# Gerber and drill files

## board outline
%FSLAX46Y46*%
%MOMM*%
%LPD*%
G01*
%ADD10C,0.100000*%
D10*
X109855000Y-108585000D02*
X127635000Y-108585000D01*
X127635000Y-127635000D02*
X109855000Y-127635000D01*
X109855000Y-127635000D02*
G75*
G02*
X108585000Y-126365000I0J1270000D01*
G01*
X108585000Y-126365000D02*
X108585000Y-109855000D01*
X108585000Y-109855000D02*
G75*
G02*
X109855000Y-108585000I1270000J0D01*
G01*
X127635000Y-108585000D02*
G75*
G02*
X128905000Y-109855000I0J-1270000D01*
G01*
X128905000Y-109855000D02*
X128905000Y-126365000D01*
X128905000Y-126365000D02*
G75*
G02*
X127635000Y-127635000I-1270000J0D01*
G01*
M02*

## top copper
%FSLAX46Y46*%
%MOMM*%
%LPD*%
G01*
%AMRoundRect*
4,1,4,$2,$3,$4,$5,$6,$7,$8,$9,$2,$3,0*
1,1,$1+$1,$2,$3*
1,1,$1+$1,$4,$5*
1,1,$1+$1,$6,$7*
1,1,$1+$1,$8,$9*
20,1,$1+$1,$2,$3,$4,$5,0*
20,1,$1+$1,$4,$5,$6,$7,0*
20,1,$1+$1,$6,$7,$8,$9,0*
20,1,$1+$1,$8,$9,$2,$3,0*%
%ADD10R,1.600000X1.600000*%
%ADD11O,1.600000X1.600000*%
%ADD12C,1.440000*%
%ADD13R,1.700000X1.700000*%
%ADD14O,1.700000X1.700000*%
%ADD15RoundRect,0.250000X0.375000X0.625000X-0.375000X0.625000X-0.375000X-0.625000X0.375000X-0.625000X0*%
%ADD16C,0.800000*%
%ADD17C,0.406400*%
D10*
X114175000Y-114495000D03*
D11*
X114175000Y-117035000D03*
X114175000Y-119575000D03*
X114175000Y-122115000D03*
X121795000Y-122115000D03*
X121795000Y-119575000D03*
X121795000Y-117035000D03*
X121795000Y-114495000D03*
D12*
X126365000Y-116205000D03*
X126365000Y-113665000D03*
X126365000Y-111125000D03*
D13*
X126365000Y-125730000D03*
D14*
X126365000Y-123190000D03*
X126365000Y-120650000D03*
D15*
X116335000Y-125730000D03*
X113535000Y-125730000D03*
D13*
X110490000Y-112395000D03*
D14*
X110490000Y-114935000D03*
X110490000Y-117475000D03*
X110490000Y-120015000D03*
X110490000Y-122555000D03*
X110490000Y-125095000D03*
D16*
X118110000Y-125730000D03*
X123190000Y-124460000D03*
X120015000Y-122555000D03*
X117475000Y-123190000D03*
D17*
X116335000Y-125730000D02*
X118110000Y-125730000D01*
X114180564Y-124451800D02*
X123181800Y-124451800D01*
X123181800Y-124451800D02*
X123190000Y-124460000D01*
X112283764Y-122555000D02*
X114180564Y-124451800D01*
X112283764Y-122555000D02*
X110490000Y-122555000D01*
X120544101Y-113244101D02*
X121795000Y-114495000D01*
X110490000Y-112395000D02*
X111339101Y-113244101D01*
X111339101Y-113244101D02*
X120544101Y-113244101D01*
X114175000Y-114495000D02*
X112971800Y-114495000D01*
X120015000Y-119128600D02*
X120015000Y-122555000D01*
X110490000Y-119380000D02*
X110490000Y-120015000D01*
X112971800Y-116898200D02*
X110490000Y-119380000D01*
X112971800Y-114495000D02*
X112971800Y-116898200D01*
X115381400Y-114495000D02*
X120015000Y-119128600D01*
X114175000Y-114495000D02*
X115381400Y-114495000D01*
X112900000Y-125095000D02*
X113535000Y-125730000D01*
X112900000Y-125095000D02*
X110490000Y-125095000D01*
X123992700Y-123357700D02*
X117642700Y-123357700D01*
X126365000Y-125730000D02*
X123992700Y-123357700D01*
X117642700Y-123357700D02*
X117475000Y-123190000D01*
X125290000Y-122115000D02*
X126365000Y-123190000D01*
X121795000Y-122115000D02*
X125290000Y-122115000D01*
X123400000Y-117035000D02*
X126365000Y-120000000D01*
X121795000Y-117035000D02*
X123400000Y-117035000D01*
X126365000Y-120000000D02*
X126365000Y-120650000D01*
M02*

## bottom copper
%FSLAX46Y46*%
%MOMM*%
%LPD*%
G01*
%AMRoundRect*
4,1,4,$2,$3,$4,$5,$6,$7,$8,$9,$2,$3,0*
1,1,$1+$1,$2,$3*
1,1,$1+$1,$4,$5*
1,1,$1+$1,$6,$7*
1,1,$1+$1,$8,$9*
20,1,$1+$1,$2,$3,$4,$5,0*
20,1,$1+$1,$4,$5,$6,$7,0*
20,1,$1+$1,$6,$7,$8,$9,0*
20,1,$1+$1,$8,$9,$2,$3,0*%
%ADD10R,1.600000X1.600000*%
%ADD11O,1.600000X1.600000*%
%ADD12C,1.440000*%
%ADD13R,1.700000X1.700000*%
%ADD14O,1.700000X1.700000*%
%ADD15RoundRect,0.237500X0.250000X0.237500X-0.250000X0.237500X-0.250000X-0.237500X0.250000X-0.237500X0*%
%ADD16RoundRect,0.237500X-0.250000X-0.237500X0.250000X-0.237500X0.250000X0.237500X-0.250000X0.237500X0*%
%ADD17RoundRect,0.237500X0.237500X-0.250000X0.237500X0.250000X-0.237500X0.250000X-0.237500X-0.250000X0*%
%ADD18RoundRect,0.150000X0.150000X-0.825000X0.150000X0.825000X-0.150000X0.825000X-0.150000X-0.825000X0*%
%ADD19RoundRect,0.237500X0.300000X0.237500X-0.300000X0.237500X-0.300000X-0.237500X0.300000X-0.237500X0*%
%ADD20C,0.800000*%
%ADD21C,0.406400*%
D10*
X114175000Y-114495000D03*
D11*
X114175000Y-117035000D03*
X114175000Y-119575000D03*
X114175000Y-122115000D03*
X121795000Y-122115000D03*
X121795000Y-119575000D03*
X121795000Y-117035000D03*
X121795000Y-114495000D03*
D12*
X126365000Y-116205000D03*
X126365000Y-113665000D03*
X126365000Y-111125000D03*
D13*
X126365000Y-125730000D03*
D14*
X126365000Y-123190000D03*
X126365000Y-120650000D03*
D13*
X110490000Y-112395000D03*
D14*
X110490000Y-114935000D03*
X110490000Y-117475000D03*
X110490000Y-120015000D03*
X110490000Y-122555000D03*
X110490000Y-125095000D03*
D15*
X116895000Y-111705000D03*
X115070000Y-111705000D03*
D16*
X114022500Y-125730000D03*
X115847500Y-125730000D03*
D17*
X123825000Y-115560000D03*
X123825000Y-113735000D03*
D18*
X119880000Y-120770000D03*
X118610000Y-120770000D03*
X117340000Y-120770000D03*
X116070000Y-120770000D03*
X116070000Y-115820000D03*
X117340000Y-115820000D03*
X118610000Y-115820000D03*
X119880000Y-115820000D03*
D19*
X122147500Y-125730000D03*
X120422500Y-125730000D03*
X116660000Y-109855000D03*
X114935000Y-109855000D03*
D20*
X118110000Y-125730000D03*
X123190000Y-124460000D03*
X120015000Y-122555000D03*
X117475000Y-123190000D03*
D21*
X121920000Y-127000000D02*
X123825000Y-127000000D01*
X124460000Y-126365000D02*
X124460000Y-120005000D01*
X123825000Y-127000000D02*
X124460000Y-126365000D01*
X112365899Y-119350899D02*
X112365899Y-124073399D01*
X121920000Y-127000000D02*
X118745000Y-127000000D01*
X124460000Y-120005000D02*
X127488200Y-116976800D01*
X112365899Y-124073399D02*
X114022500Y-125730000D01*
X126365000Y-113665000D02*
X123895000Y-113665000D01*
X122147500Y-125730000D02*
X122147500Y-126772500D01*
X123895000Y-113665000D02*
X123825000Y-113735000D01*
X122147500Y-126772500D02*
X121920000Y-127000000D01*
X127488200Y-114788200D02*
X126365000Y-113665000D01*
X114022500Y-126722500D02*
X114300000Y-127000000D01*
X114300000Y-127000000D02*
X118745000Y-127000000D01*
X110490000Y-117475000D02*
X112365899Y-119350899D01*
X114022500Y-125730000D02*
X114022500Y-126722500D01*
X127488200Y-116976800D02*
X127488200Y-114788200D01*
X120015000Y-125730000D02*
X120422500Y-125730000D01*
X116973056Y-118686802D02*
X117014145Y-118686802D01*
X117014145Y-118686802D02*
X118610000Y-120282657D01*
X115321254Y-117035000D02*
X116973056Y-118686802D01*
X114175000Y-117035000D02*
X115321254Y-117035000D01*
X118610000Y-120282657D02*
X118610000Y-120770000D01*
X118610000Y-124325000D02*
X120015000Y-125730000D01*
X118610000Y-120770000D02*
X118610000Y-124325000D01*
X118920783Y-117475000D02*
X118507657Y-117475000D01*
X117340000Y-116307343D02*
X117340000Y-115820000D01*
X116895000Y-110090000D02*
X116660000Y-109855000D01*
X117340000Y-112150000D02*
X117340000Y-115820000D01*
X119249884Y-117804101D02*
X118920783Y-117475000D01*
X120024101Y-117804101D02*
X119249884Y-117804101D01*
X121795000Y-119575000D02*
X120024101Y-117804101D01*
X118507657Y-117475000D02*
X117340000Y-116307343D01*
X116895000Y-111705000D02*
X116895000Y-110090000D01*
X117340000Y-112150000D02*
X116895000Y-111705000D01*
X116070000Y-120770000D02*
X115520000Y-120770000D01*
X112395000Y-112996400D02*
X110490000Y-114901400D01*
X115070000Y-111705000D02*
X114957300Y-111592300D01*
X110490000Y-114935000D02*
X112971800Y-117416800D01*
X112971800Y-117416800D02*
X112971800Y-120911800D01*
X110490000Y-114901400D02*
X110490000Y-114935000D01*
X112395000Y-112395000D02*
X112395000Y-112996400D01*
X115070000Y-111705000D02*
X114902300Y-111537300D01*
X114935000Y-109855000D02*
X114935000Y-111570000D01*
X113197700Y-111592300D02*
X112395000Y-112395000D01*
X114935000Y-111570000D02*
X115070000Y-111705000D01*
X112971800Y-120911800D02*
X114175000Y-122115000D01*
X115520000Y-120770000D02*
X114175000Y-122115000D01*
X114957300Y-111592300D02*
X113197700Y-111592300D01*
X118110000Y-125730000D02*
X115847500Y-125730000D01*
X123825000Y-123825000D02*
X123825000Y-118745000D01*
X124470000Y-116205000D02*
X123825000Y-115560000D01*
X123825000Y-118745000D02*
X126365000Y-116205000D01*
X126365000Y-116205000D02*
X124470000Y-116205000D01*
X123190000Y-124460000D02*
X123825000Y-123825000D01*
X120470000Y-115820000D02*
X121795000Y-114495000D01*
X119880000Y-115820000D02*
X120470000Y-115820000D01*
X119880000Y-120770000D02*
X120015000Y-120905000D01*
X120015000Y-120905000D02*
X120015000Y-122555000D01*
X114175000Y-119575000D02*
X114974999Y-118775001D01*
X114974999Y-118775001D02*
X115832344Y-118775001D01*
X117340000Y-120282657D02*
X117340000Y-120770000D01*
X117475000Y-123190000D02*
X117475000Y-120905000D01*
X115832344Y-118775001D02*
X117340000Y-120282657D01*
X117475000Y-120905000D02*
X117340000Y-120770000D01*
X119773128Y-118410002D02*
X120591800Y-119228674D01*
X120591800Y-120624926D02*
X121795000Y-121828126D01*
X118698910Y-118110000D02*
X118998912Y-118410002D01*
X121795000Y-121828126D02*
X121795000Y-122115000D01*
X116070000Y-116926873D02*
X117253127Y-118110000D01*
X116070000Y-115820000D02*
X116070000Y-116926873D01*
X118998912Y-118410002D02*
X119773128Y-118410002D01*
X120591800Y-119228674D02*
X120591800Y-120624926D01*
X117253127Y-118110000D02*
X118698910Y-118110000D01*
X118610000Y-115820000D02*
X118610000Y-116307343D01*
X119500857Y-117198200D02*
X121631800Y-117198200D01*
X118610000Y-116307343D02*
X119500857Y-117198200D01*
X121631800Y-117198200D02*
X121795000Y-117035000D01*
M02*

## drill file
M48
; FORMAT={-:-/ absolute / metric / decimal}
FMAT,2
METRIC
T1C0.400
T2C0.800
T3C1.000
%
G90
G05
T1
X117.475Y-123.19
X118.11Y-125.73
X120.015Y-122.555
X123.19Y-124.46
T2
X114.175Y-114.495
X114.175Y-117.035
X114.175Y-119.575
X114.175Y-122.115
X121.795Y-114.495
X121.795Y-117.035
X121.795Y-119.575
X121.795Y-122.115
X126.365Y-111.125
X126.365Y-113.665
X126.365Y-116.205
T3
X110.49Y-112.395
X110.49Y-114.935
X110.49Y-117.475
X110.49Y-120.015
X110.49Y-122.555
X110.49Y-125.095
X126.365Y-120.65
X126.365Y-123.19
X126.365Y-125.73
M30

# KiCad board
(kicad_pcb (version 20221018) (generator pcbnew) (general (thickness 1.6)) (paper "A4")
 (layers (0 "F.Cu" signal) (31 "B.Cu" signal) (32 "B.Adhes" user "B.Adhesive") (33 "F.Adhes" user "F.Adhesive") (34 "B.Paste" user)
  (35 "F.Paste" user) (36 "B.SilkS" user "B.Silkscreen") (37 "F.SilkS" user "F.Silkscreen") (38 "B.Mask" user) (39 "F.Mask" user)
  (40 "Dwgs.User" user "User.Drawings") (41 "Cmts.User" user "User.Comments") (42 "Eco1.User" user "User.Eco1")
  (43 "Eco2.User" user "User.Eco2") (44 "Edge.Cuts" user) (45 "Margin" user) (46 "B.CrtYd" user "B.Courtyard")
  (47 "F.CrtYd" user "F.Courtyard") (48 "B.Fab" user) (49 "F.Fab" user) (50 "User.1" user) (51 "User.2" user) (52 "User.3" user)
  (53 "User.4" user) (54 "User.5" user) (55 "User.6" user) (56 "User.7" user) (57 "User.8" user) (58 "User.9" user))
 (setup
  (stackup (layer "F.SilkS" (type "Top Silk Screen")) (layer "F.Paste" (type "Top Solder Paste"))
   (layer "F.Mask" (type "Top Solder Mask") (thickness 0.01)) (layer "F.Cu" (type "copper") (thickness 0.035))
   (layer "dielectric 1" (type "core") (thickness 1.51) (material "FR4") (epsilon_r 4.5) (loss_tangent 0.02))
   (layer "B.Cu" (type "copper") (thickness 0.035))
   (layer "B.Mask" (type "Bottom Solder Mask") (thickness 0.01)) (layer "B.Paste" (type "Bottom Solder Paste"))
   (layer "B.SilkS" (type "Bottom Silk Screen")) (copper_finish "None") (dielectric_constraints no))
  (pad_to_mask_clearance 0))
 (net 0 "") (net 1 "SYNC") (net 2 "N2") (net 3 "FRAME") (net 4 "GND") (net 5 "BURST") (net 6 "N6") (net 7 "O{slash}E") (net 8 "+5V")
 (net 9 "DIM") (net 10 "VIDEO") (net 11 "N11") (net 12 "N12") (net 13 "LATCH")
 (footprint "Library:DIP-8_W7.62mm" (layer "F.Cu") (at 114.175 114.495)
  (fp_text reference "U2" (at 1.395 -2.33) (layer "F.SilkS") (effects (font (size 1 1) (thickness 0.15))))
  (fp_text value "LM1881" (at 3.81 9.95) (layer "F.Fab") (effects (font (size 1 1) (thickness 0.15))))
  (pad "1" thru_hole rect (at 0 0) (size 1.6 1.6) (drill 0.8) (layers "*.Cu" "*.Mask") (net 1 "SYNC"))
  (pad "2" thru_hole oval (at 0 2.54) (size 1.6 1.6) (drill 0.8) (layers "*.Cu" "*.Mask") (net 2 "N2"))
  (pad "3" thru_hole oval (at 0 5.08) (size 1.6 1.6) (drill 0.8) (layers "*.Cu" "*.Mask") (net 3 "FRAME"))
  (pad "4" thru_hole oval (at 0 7.62) (size 1.6 1.6) (drill 0.8) (layers "*.Cu" "*.Mask") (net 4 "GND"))
  (pad "5" thru_hole oval (at 7.62 7.62) (size 1.6 1.6) (drill 0.8) (layers "*.Cu" "*.Mask") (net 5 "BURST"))
  (pad "6" thru_hole oval (at 7.62 5.08) (size 1.6 1.6) (drill 0.8) (layers "*.Cu" "*.Mask") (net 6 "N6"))
  (pad "7" thru_hole oval (at 7.62 2.54) (size 1.6 1.6) (drill 0.8) (layers "*.Cu" "*.Mask") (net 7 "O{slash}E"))
  (pad "8" thru_hole oval (at 7.62 0) (size 1.6 1.6) (drill 0.8) (layers "*.Cu" "*.Mask") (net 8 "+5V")))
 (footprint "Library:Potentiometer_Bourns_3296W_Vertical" (layer "F.Cu") (at 126.365 116.205 -90)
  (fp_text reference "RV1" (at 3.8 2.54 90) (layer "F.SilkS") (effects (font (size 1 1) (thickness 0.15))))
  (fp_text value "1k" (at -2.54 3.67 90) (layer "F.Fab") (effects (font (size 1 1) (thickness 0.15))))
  (pad "1" thru_hole circle (at 0 0 270) (size 1.44 1.44) (drill 0.8) (layers "*.Cu" "*.Mask") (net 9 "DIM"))
  (pad "2" thru_hole circle (at -2.54 0 270) (size 1.44 1.44) (drill 0.8) (layers "*.Cu" "*.Mask") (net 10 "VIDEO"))
  (pad "3" thru_hole circle (at -5.08 0 270) (size 1.44 1.44) (drill 0.8) (layers "*.Cu" "*.Mask") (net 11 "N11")))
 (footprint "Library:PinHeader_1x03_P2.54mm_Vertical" (layer "F.Cu") (at 126.365 125.73 180)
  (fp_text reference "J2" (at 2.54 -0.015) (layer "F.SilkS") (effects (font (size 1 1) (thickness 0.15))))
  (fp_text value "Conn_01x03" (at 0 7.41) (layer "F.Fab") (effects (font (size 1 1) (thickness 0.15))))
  (pad "1" thru_hole rect (at 0 0 180) (size 1.7 1.7) (drill 1) (layers "*.Cu" "*.Mask") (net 3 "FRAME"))
  (pad "2" thru_hole oval (at 0 2.54 180) (size 1.7 1.7) (drill 1) (layers "*.Cu" "*.Mask") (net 5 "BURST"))
  (pad "3" thru_hole oval (at 0 5.08 180) (size 1.7 1.7) (drill 1) (layers "*.Cu" "*.Mask") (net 7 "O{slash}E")))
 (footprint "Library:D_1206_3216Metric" (layer "F.Cu") (at 114.935 125.73 180)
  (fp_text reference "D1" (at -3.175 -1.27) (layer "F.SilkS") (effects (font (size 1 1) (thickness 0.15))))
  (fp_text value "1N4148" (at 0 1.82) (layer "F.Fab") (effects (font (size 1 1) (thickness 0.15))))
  (pad "1" smd roundrect (at -1.4 0 180) (size 1.25 1.75) (layers "F.Cu" "F.Paste" "F.Mask") (roundrect_rratio 0.2) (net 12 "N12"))
  (pad "2" smd roundrect (at 1.4 0 180) (size 1.25 1.75) (layers "F.Cu" "F.Paste" "F.Mask") (roundrect_rratio 0.2) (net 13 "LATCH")))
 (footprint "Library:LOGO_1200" (layer "F.Cu") (at 121.285 110.49)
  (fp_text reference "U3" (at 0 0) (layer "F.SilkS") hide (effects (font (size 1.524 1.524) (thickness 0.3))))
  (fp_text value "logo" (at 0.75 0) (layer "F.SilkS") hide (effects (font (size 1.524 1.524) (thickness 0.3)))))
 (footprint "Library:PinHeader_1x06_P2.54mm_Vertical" (layer "F.Cu") (at 110.49 112.395)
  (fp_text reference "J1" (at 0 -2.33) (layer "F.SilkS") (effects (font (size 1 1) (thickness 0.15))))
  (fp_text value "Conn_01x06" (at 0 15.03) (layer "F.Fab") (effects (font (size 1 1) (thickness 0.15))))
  (pad "1" thru_hole rect (at 0 0) (size 1.7 1.7) (drill 1) (layers "*.Cu" "*.Mask") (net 8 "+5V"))
  (pad "2" thru_hole oval (at 0 2.54) (size 1.7 1.7) (drill 1) (layers "*.Cu" "*.Mask") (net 4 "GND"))
  (pad "3" thru_hole oval (at 0 5.08) (size 1.7 1.7) (drill 1) (layers "*.Cu" "*.Mask") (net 10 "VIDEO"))
  (pad "4" thru_hole oval (at 0 7.62) (size 1.7 1.7) (drill 1) (layers "*.Cu" "*.Mask") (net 1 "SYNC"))
  (pad "5" thru_hole oval (at 0 10.16) (size 1.7 1.7) (drill 1) (layers "*.Cu" "*.Mask") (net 9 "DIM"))
  (pad "6" thru_hole oval (at 0 12.7) (size 1.7 1.7) (drill 1) (layers "*.Cu" "*.Mask") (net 13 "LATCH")))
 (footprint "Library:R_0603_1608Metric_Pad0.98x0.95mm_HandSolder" (layer "B.Cu") (at 115.9825 111.705 180)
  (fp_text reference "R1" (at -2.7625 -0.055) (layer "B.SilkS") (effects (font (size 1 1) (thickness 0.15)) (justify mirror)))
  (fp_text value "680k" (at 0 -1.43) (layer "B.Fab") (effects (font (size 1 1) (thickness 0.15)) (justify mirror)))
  (pad "1" smd roundrect (at -0.9125 0 180) (size 0.975 0.95) (layers "B.Cu" "B.Paste" "B.Mask") (roundrect_rratio 0.25) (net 6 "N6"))
  (pad "2" smd roundrect (at 0.9125 0 180) (size 0.975 0.95) (layers "B.Cu" "B.Paste" "B.Mask") (roundrect_rratio 0.25) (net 4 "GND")))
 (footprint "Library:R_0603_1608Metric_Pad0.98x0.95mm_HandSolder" (layer "B.Cu") (at 114.935 125.73)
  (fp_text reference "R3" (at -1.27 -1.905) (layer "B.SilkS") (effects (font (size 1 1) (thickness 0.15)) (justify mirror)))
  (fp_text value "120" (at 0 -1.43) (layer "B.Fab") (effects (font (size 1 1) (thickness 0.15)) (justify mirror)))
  (pad "1" smd roundrect (at -0.9125 0) (size 0.975 0.95) (layers "B.Cu" "B.Paste" "B.Mask") (roundrect_rratio 0.25) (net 10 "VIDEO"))
  (pad "2" smd roundrect (at 0.9125 0) (size 0.975 0.95) (layers "B.Cu" "B.Paste" "B.Mask") (roundrect_rratio 0.25) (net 12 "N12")))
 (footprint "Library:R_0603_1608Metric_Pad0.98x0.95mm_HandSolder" (layer "B.Cu") (at 123.825 114.6475 90)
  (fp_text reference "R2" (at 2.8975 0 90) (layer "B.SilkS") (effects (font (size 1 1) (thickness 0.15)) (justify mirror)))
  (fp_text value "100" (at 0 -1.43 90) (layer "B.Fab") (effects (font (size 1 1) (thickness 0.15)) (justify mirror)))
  (pad "1" smd roundrect (at -0.9125 0 90) (size 0.975 0.95) (layers "B.Cu" "B.Paste" "B.Mask") (roundrect_rratio 0.25) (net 9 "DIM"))
  (pad "2" smd roundrect (at 0.9125 0 90) (size 0.975 0.95) (layers "B.Cu" "B.Paste" "B.Mask") (roundrect_rratio 0.25) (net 10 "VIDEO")))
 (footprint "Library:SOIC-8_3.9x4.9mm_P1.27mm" (layer "B.Cu") (at 117.975 118.295 90)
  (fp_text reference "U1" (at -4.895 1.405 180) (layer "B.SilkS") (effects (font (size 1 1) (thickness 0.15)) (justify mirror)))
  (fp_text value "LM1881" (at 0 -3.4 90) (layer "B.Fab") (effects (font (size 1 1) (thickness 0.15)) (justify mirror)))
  (pad "1" smd roundrect (at -2.475 1.905 90) (size 1.95 0.6) (layers "B.Cu" "B.Paste" "B.Mask") (roundrect_rratio 0.25) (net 1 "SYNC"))
  (pad "2" smd roundrect (at -2.475 0.635 90) (size 1.95 0.6) (layers "B.Cu" "B.Paste" "B.Mask") (roundrect_rratio 0.25) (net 2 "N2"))
  (pad "3" smd roundrect (at -2.475 -0.635 90) (size 1.95 0.6) (layers "B.Cu" "B.Paste" "B.Mask") (roundrect_rratio 0.25) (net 3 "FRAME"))
  (pad "4" smd roundrect (at -2.475 -1.905 90) (size 1.95 0.6) (layers "B.Cu" "B.Paste" "B.Mask") (roundrect_rratio 0.25) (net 4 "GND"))
  (pad "5" smd roundrect (at 2.475 -1.905 90) (size 1.95 0.6) (layers "B.Cu" "B.Paste" "B.Mask") (roundrect_rratio 0.25) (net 5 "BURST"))
  (pad "6" smd roundrect (at 2.475 -0.635 90) (size 1.95 0.6) (layers "B.Cu" "B.Paste" "B.Mask") (roundrect_rratio 0.25) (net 6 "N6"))
  (pad "7" smd roundrect (at 2.475 0.635 90) (size 1.95 0.6) (layers "B.Cu" "B.Paste" "B.Mask") (roundrect_rratio 0.25) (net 7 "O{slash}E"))
  (pad "8" smd roundrect (at 2.475 1.905 90) (size 1.95 0.6) (layers "B.Cu" "B.Paste" "B.Mask") (roundrect_rratio 0.25) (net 8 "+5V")))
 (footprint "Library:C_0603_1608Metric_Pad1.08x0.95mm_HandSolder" (layer "B.Cu") (at 121.285 125.73 180)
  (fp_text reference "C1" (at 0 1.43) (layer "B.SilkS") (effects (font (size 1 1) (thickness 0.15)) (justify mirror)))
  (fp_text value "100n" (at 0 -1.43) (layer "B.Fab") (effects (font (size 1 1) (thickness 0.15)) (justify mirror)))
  (pad "1" smd roundrect (at -0.8625 0 180) (size 1.075 0.95) (layers "B.Cu" "B.Paste" "B.Mask") (roundrect_rratio 0.25) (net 10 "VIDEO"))
  (pad "2" smd roundrect (at 0.8625 0 180) (size 1.075 0.95) (layers "B.Cu" "B.Paste" "B.Mask") (roundrect_rratio 0.25) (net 2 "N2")))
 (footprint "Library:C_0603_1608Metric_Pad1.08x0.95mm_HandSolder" (layer "B.Cu") (at 115.7975 109.855 180)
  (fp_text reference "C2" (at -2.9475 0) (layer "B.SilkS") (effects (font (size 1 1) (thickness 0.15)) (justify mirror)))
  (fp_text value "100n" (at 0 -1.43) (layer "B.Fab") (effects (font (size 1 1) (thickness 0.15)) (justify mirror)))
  (pad "1" smd roundrect (at -0.8625 0 180) (size 1.075 0.95) (layers "B.Cu" "B.Paste" "B.Mask") (roundrect_rratio 0.25) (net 6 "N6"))
  (pad "2" smd roundrect (at 0.8625 0 180) (size 1.075 0.95) (layers "B.Cu" "B.Paste" "B.Mask") (roundrect_rratio 0.25) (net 4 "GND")))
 (gr_line (start 109.855 108.585) (end 127.635 108.585) (stroke (width 0.1) (type solid)) (layer "Edge.Cuts"))
 (gr_line (start 127.635 127.635) (end 109.855 127.635) (stroke (width 0.1) (type solid)) (layer "Edge.Cuts"))
 (gr_arc (start 109.855 127.635) (mid 108.956974 127.263026) (end 108.585 126.365) (stroke (width 0.1) (type solid)) (layer "Edge.Cuts"))
 (gr_line (start 108.585 126.365) (end 108.585 109.855) (stroke (width 0.1) (type solid)) (layer "Edge.Cuts"))
 (gr_arc (start 108.585 109.855) (mid 108.956974 108.956974) (end 109.855 108.585) (stroke (width 0.1) (type solid)) (layer "Edge.Cuts"))
 (gr_arc (start 127.635 108.585) (mid 128.533026 108.956974) (end 128.905 109.855) (stroke (width 0.1) (type solid)) (layer "Edge.Cuts"))
 (gr_line (start 128.905 109.855) (end 128.905 126.365) (stroke (width 0.1) (type solid)) (layer "Edge.Cuts"))
 (gr_arc (start 128.905 126.365) (mid 128.533026 127.263026) (end 127.635 127.635) (stroke (width 0.1) (type solid)) (layer "Edge.Cuts"))
 (segment (start 121.92 127) (end 123.825 127) (width 0.4064) (layer "B.Cu") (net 10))
 (segment (start 124.46 126.365) (end 124.46 120.005) (width 0.4064) (layer "B.Cu") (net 10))
 (segment (start 123.825 127) (end 124.46 126.365) (width 0.4064) (layer "B.Cu") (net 10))
 (segment (start 112.365899 119.350899) (end 112.365899 124.073399) (width 0.4064) (layer "B.Cu") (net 10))
 (segment (start 121.92 127) (end 118.745 127) (width 0.4064) (layer "B.Cu") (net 10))
 (segment (start 124.46 120.005) (end 127.4882 116.9768) (width 0.4064) (layer "B.Cu") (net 10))
 (segment (start 112.365899 124.073399) (end 114.0225 125.73) (width 0.4064) (layer "B.Cu") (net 10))
 (segment (start 126.365 113.665) (end 123.895 113.665) (width 0.4064) (layer "B.Cu") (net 10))
 (segment (start 122.1475 125.73) (end 122.1475 126.7725) (width 0.4064) (layer "B.Cu") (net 10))
 (segment (start 123.895 113.665) (end 123.825 113.735) (width 0.4064) (layer "B.Cu") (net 10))
 (segment (start 122.1475 126.7725) (end 121.92 127) (width 0.4064) (layer "B.Cu") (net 10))
 (segment (start 127.4882 114.7882) (end 126.365 113.665) (width 0.4064) (layer "B.Cu") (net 10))
 (segment (start 114.0225 126.7225) (end 114.3 127) (width 0.4064) (layer "B.Cu") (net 10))
 (segment (start 114.3 127) (end 118.745 127) (width 0.4064) (layer "B.Cu") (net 10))
 (segment (start 110.49 117.475) (end 112.365899 119.350899) (width 0.4064) (layer "B.Cu") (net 10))
 (segment (start 114.0225 125.73) (end 114.0225 126.7225) (width 0.4064) (layer "B.Cu") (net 10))
 (segment (start 127.4882 116.9768) (end 127.4882 114.7882) (width 0.4064) (layer "B.Cu") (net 10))
 (segment (start 120.015 125.73) (end 120.4225 125.73) (width 0.4064) (layer "B.Cu") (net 2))
 (segment (start 116.973056 118.686802) (end 117.014145 118.686802) (width 0.4064) (layer "B.Cu") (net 2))
 (segment (start 117.014145 118.686802) (end 118.61 120.282657) (width 0.4064) (layer "B.Cu") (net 2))
 (segment (start 115.321254 117.035) (end 116.973056 118.686802) (width 0.4064) (layer "B.Cu") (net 2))
 (segment (start 114.175 117.035) (end 115.321254 117.035) (width 0.4064) (layer "B.Cu") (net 2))
 (segment (start 118.61 120.282657) (end 118.61 120.77) (width 0.4064) (layer "B.Cu") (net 2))
 (segment (start 118.61 124.325) (end 120.015 125.73) (width 0.4064) (layer "B.Cu") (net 2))
 (segment (start 118.61 120.77) (end 118.61 124.325) (width 0.4064) (layer "B.Cu") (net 2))
 (segment (start 118.920783 117.475) (end 118.507657 117.475) (width 0.4064) (layer "B.Cu") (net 6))
 (segment (start 117.34 116.307343) (end 117.34 115.82) (width 0.4064) (layer "B.Cu") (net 6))
 (segment (start 116.895 110.09) (end 116.66 109.855) (width 0.4064) (layer "B.Cu") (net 6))
 (segment (start 117.34 112.15) (end 117.34 115.82) (width 0.4064) (layer "B.Cu") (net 6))
 (segment (start 119.249884 117.804101) (end 118.920783 117.475) (width 0.4064) (layer "B.Cu") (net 6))
 (segment (start 120.024101 117.804101) (end 119.249884 117.804101) (width 0.4064) (layer "B.Cu") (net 6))
 (segment (start 121.795 119.575) (end 120.024101 117.804101) (width 0.4064) (layer "B.Cu") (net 6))
 (segment (start 118.507657 117.475) (end 117.34 116.307343) (width 0.4064) (layer "B.Cu") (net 6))
 (segment (start 116.895 111.705) (end 116.895 110.09) (width 0.4064) (layer "B.Cu") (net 6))
 (segment (start 117.34 112.15) (end 116.895 111.705) (width 0.4064) (layer "B.Cu") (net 6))
 (segment (start 116.07 120.77) (end 115.52 120.77) (width 0.4064) (layer "B.Cu") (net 4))
 (segment (start 112.395 112.9964) (end 110.49 114.9014) (width 0.4064) (layer "B.Cu") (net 4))
 (segment (start 115.07 111.705) (end 114.9573 111.5923) (width 0.4064) (layer "B.Cu") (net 4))
 (segment (start 110.49 114.935) (end 112.9718 117.4168) (width 0.4064) (layer "B.Cu") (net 4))
 (segment (start 112.9718 117.4168) (end 112.9718 120.9118) (width 0.4064) (layer "B.Cu") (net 4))
 (segment (start 110.49 114.9014) (end 110.49 114.935) (width 0.4064) (layer "B.Cu") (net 4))
 (segment (start 112.395 112.395) (end 112.395 112.9964) (width 0.4064) (layer "B.Cu") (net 4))
 (segment (start 115.07 111.705) (end 114.9023 111.5373) (width 0.4064) (layer "B.Cu") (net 4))
 (segment (start 114.935 109.855) (end 114.935 111.57) (width 0.4064) (layer "B.Cu") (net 4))
 (segment (start 113.1977 111.5923) (end 112.395 112.395) (width 0.4064) (layer "B.Cu") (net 4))
 (segment (start 114.935 111.57) (end 115.07 111.705) (width 0.4064) (layer "B.Cu") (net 4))
 (segment (start 112.9718 120.9118) (end 114.175 122.115) (width 0.4064) (layer "B.Cu") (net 4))
 (segment (start 115.52 120.77) (end 114.175 122.115) (width 0.4064) (layer "B.Cu") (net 4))
 (segment (start 114.9573 111.5923) (end 113.1977 111.5923) (width 0.4064) (layer "B.Cu") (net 4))
 (segment (start 116.335 125.73) (end 118.11 125.73) (width 0.4064) (layer "F.Cu") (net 12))
 (via (at 118.11 125.73) (size 0.8) (drill 0.4) (layers "F.Cu" "B.Cu") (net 12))
 (segment (start 118.11 125.73) (end 115.8475 125.73) (width 0.4064) (layer "B.Cu") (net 12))
 (segment (start 114.180564 124.4518) (end 123.1818 124.4518) (width 0.4064) (layer "F.Cu") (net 9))
 (segment (start 123.1818 124.4518) (end 123.19 124.46) (width 0.4064) (layer "F.Cu") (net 9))
 (segment (start 112.283764 122.555) (end 114.180564 124.4518) (width 0.4064) (layer "F.Cu") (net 9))
 (segment (start 112.283764 122.555) (end 110.49 122.555) (width 0.4064) (layer "F.Cu") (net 9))
 (via (at 123.19 124.46) (size 0.8) (drill 0.4) (layers "F.Cu" "B.Cu") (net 9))
 (segment (start 123.825 123.825) (end 123.825 118.745) (width 0.4064) (layer "B.Cu") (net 9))
 (segment (start 124.47 116.205) (end 123.825 115.56) (width 0.4064) (layer "B.Cu") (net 9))
 (segment (start 123.825 118.745) (end 126.365 116.205) (width 0.4064) (layer "B.Cu") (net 9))
 (segment (start 126.365 116.205) (end 124.47 116.205) (width 0.4064) (layer "B.Cu") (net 9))
 (segment (start 123.19 124.46) (end 123.825 123.825) (width 0.4064) (layer "B.Cu") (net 9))
 (segment (start 120.544101 113.244101) (end 121.795 114.495) (width 0.4064) (layer "F.Cu") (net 8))
 (segment (start 110.49 112.395) (end 111.339101 113.244101) (width 0.4064) (layer "F.Cu") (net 8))
 (segment (start 111.339101 113.244101) (end 120.544101 113.244101) (width 0.4064) (layer "F.Cu") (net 8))
 (segment (start 120.47 115.82) (end 121.795 114.495) (width 0.4064) (layer "B.Cu") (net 8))
 (segment (start 119.88 115.82) (end 120.47 115.82) (width 0.4064) (layer "B.Cu") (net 8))
 (segment (start 114.175 114.495) (end 112.9718 114.495) (width 0.4064) (layer "F.Cu") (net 1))
 (segment (start 120.015 119.1286) (end 120.015 122.555) (width 0.4064) (layer "F.Cu") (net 1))
 (segment (start 110.49 119.38) (end 110.49 120.015) (width 0.4064) (layer "F.Cu") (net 1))
 (segment (start 112.9718 116.8982) (end 110.49 119.38) (width 0.4064) (layer "F.Cu") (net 1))
 (segment (start 112.9718 114.495) (end 112.9718 116.8982) (width 0.4064) (layer "F.Cu") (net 1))
 (segment (start 115.3814 114.495) (end 120.015 119.1286) (width 0.4064) (layer "F.Cu") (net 1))
 (segment (start 114.175 114.495) (end 115.3814 114.495) (width 0.4064) (layer "F.Cu") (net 1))
 (via (at 120.015 122.555) (size 0.8) (drill 0.4) (layers "F.Cu" "B.Cu") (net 1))
 (segment (start 119.88 120.77) (end 120.015 120.905) (width 0.4064) (layer "B.Cu") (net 1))
 (segment (start 120.015 120.905) (end 120.015 122.555) (width 0.4064) (layer "B.Cu") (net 1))
 (segment (start 112.9 125.095) (end 113.535 125.73) (width 0.4064) (layer "F.Cu") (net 13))
 (segment (start 112.9 125.095) (end 110.49 125.095) (width 0.4064) (layer "F.Cu") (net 13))
 (segment (start 123.9927 123.3577) (end 117.6427 123.3577) (width 0.4064) (layer "F.Cu") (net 3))
 (segment (start 126.365 125.73) (end 123.9927 123.3577) (width 0.4064) (layer "F.Cu") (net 3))
 (segment (start 117.6427 123.3577) (end 117.475 123.19) (width 0.4064) (layer "F.Cu") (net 3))
 (via (at 117.475 123.19) (size 0.8) (drill 0.4) (layers "F.Cu" "B.Cu") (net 3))
 (segment (start 114.175 119.575) (end 114.974999 118.775001) (width 0.4064) (layer "B.Cu") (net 3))
 (segment (start 114.974999 118.775001) (end 115.832344 118.775001) (width 0.4064) (layer "B.Cu") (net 3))
 (segment (start 117.34 120.282657) (end 117.34 120.77) (width 0.4064) (layer "B.Cu") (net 3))
 (segment (start 117.475 123.19) (end 117.475 120.905) (width 0.4064) (layer "B.Cu") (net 3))
 (segment (start 115.832344 118.775001) (end 117.34 120.282657) (width 0.4064) (layer "B.Cu") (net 3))
 (segment (start 117.475 120.905) (end 117.34 120.77) (width 0.4064) (layer "B.Cu") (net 3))
 (segment (start 125.29 122.115) (end 126.365 123.19) (width 0.4064) (layer "F.Cu") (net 5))
 (segment (start 121.795 122.115) (end 125.29 122.115) (width 0.4064) (layer "F.Cu") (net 5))
 (segment (start 119.773128 118.410002) (end 120.5918 119.228674) (width 0.4064) (layer "B.Cu") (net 5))
 (segment (start 120.5918 120.624926) (end 121.795 121.828126) (width 0.4064) (layer "B.Cu") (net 5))
 (segment (start 118.69891 118.11) (end 118.998912 118.410002) (width 0.4064) (layer "B.Cu") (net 5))
 (segment (start 121.795 121.828126) (end 121.795 122.115) (width 0.4064) (layer "B.Cu") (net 5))
 (segment (start 116.07 116.926873) (end 117.253127 118.11) (width 0.4064) (layer "B.Cu") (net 5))
 (segment (start 116.07 115.82) (end 116.07 116.926873) (width 0.4064) (layer "B.Cu") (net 5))
 (segment (start 118.998912 118.410002) (end 119.773128 118.410002) (width 0.4064) (layer "B.Cu") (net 5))
 (segment (start 120.5918 119.228674) (end 120.5918 120.624926) (width 0.4064) (layer "B.Cu") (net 5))
 (segment (start 117.253127 118.11) (end 118.69891 118.11) (width 0.4064) (layer "B.Cu") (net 5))
 (segment (start 123.4 117.035) (end 126.365 120) (width 0.4064) (layer "F.Cu") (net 7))
 (segment (start 121.795 117.035) (end 123.4 117.035) (width 0.4064) (layer "F.Cu") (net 7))
 (segment (start 126.365 120) (end 126.365 120.65) (width 0.4064) (layer "F.Cu") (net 7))
 (segment (start 118.61 115.82) (end 118.61 116.307343) (width 0.4064) (layer "B.Cu") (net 7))
 (segment (start 119.500857 117.1982) (end 121.6318 117.1982) (width 0.4064) (layer "B.Cu") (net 7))
 (segment (start 118.61 116.307343) (end 119.500857 117.1982) (width 0.4064) (layer "B.Cu") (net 7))
 (segment (start 121.6318 117.1982) (end 121.795 117.035) (width 0.4064) (layer "B.Cu") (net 7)))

